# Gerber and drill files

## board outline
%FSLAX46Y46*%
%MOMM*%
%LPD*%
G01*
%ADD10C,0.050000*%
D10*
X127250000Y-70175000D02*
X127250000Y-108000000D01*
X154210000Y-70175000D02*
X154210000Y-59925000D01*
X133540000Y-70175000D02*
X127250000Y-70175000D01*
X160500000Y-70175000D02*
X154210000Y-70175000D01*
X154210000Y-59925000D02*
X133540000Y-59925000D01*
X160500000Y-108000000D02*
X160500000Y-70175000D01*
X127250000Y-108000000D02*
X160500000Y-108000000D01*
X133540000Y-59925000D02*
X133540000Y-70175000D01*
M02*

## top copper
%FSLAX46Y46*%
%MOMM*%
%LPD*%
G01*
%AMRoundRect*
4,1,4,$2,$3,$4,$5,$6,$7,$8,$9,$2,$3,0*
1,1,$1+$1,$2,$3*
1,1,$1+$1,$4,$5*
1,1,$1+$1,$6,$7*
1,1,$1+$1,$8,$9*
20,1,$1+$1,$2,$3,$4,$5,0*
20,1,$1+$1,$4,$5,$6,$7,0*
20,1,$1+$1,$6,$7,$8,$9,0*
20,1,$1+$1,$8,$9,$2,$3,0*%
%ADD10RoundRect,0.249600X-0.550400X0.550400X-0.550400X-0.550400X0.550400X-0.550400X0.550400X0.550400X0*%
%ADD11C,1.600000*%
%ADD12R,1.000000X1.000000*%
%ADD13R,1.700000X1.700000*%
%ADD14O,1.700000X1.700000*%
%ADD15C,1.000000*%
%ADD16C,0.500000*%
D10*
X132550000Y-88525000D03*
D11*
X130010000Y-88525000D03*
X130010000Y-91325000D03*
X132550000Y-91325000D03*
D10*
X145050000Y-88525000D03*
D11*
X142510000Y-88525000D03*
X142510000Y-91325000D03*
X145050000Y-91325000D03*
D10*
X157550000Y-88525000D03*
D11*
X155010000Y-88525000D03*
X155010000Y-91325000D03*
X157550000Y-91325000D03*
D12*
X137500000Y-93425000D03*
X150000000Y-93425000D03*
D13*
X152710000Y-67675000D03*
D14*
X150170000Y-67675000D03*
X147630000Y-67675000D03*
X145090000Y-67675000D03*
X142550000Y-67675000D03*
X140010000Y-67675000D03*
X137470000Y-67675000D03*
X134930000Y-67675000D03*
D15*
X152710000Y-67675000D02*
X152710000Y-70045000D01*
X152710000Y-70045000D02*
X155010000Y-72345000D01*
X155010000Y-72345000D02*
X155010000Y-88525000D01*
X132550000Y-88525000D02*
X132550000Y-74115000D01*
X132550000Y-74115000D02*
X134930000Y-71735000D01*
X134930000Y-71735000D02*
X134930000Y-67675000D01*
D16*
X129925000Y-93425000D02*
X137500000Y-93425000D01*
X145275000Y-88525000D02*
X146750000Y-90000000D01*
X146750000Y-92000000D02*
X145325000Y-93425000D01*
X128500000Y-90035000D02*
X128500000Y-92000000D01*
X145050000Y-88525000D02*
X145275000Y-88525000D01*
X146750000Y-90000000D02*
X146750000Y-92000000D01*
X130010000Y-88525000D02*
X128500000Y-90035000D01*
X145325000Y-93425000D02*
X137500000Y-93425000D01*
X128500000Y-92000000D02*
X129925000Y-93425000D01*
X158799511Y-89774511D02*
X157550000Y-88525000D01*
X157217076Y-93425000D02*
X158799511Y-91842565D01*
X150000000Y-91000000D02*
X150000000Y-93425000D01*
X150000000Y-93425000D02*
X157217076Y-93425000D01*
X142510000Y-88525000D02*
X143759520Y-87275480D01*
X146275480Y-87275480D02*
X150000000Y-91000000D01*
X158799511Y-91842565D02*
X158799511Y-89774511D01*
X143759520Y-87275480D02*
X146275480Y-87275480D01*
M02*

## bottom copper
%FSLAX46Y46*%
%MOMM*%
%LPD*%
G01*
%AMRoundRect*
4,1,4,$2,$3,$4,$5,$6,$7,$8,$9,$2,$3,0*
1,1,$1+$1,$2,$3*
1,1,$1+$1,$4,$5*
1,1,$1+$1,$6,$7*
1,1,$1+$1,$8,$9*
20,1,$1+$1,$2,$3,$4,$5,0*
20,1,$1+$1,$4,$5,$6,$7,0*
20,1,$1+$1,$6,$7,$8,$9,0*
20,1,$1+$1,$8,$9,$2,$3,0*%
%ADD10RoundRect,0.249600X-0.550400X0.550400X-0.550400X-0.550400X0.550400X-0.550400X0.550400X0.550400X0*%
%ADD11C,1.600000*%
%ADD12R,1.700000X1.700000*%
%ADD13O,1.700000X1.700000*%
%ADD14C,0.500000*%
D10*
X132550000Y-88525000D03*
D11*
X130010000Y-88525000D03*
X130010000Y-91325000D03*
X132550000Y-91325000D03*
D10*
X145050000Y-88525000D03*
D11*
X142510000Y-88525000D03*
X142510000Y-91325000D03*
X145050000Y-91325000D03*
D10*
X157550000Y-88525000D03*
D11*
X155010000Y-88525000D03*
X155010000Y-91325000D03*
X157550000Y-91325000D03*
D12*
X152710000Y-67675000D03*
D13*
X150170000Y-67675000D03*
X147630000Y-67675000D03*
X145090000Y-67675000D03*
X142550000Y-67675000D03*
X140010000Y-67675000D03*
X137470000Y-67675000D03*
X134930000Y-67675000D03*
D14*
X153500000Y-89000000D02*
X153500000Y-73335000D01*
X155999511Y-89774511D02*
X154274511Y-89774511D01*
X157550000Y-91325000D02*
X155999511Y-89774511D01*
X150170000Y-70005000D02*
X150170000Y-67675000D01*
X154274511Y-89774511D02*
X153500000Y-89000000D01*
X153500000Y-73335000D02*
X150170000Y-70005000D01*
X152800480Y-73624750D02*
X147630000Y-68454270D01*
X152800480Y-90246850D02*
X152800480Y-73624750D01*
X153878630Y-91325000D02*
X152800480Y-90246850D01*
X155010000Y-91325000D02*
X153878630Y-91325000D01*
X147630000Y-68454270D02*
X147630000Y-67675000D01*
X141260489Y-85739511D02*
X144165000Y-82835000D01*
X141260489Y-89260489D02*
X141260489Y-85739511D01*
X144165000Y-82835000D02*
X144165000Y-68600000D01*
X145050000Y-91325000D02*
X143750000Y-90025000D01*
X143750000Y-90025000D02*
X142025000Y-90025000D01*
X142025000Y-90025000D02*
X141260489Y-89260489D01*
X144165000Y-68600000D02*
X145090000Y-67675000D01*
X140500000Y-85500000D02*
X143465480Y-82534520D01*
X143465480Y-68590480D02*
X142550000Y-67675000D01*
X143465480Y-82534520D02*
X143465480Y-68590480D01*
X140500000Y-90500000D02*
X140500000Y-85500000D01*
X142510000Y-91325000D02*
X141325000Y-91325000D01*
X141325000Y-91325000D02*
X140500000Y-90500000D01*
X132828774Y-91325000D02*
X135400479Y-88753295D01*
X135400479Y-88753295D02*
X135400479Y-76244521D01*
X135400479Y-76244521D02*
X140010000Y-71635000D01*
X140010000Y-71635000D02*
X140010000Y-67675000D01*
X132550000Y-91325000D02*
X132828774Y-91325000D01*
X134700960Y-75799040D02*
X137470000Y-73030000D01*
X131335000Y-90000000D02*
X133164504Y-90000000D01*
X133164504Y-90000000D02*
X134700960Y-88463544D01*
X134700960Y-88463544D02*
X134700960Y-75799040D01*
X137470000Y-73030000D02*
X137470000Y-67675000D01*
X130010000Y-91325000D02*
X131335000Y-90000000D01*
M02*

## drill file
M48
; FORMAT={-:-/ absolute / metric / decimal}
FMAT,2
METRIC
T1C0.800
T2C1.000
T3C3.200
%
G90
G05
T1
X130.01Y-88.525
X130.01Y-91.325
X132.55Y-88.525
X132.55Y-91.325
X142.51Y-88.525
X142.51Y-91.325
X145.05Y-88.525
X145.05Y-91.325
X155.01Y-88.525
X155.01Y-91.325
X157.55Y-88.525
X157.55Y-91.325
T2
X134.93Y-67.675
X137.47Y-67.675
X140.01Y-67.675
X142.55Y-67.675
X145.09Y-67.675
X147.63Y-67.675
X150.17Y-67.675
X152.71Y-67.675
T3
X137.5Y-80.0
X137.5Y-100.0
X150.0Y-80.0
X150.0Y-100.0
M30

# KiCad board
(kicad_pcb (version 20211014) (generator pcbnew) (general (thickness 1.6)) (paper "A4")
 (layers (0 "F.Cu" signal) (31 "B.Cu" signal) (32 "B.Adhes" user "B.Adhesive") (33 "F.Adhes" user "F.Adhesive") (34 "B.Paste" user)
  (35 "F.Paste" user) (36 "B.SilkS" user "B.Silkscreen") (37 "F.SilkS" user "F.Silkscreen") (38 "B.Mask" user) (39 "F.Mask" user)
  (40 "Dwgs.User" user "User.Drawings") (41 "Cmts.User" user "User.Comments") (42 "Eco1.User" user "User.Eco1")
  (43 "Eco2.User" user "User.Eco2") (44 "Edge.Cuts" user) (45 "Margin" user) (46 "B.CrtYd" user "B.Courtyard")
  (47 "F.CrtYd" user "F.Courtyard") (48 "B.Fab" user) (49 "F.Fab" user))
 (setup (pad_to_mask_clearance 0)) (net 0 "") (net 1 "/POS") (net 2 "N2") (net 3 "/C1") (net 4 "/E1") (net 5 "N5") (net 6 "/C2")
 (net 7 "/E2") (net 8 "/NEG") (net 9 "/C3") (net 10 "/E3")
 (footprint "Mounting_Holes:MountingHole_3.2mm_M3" (layer "F.Cu") (at 137.5 100)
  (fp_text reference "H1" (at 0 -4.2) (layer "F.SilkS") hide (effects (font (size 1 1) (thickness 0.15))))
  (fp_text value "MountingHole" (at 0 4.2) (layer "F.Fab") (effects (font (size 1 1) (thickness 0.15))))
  (pad "" np_thru_hole circle locked (at 0 0) (size 3.2 3.2) (drill 3.2) (layers *.Cu *.Mask)))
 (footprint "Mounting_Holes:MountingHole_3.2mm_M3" (layer "F.Cu") (at 137.5 80)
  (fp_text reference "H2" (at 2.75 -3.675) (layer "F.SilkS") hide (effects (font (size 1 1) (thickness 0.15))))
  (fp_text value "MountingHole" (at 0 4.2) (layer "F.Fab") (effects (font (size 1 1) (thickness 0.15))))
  (pad "" np_thru_hole circle locked (at 0 0) (size 3.2 3.2) (drill 3.2) (layers *.Cu *.Mask)))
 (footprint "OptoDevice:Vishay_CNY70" (layer "F.Cu") (at 132.55 88.525 -90)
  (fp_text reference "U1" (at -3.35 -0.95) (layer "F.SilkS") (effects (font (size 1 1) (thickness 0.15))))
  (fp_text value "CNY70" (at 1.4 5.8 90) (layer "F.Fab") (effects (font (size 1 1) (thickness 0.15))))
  (pad "1" thru_hole roundrect (at 0 0 270) (size 1.6 1.6) (drill 0.8) (layers *.Cu *.Mask) (roundrect_rratio 0.156) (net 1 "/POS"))
  (pad "2" thru_hole circle (at 0 2.54 270) (size 1.6 1.6) (drill 0.8) (layers *.Cu *.Mask) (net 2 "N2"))
  (pad "3" thru_hole circle (at 2.8 2.54 270) (size 1.6 1.6) (drill 0.8) (layers *.Cu *.Mask) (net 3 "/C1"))
  (pad "4" thru_hole circle (at 2.8 0 270) (size 1.6 1.6) (drill 0.8) (layers *.Cu *.Mask) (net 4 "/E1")))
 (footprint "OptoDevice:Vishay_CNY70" (layer "F.Cu") (at 145.05 88.525 -90)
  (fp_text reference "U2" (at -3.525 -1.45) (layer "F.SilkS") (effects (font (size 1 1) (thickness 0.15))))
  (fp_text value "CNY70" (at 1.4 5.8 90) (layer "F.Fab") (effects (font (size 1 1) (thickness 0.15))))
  (pad "1" thru_hole roundrect (at 0 0 270) (size 1.6 1.6) (drill 0.8) (layers *.Cu *.Mask) (roundrect_rratio 0.156) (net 2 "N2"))
  (pad "2" thru_hole circle (at 0 2.54 270) (size 1.6 1.6) (drill 0.8) (layers *.Cu *.Mask) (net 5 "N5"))
  (pad "3" thru_hole circle (at 2.8 2.54 270) (size 1.6 1.6) (drill 0.8) (layers *.Cu *.Mask) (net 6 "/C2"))
  (pad "4" thru_hole circle (at 2.8 0 270) (size 1.6 1.6) (drill 0.8) (layers *.Cu *.Mask) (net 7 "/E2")))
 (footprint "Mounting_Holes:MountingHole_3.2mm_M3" (layer "F.Cu") (at 150 100)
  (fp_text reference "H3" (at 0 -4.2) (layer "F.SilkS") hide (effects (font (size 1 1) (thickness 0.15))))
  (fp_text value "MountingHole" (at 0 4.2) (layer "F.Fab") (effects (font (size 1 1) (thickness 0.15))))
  (pad "" np_thru_hole circle locked (at 0 0) (size 3.2 3.2) (drill 3.2) (layers *.Cu *.Mask)))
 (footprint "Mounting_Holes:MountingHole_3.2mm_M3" (layer "F.Cu") (at 150 80)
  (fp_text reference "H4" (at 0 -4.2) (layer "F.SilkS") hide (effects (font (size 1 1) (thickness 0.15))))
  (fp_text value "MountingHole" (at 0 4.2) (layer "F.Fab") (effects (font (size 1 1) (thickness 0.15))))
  (pad "" np_thru_hole circle locked (at 0 0) (size 3.2 3.2) (drill 3.2) (layers *.Cu *.Mask)))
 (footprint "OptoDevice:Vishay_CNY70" (layer "F.Cu") (at 157.55 88.525 -90)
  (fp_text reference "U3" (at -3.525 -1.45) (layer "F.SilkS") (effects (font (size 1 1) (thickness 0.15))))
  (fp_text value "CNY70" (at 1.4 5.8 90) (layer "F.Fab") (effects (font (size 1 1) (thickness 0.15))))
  (pad "1" thru_hole roundrect (at 0 0 270) (size 1.6 1.6) (drill 0.8) (layers *.Cu *.Mask) (roundrect_rratio 0.156) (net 5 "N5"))
  (pad "2" thru_hole circle (at 0 2.54 270) (size 1.6 1.6) (drill 0.8) (layers *.Cu *.Mask) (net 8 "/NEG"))
  (pad "3" thru_hole circle (at 2.8 2.54 270) (size 1.6 1.6) (drill 0.8) (layers *.Cu *.Mask) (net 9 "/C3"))
  (pad "4" thru_hole circle (at 2.8 0 270) (size 1.6 1.6) (drill 0.8) (layers *.Cu *.Mask) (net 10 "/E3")))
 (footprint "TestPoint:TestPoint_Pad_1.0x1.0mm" (layer "F.Cu") (at 137.5 93.425)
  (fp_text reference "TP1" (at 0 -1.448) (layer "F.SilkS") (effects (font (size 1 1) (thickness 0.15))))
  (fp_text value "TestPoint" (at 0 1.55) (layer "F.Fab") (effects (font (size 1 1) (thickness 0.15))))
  (pad "1" smd rect locked (at 0 0) (size 1 1) (layers "F.Cu" "F.Mask") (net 2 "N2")))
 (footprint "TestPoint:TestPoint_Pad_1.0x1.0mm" (layer "F.Cu") (at 150 93.425)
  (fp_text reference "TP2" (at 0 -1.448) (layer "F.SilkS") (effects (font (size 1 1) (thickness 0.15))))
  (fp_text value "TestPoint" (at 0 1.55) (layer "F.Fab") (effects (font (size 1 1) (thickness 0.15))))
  (pad "1" smd rect locked (at 0 0) (size 1 1) (layers "F.Cu" "F.Mask") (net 5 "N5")))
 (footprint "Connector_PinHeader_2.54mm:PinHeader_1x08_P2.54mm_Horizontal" (layer "B.Cu") (at 152.71 67.675 90)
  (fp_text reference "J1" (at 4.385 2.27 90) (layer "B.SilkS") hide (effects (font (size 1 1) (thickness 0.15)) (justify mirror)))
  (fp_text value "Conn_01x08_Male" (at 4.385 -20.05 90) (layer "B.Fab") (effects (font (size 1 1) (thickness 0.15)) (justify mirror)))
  (pad "1" thru_hole rect (at 0 0 90) (size 1.7 1.7) (drill 1) (layers *.Cu *.Mask) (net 8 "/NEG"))
  (pad "2" thru_hole oval (at 0 -2.54 90) (size 1.7 1.7) (drill 1) (layers *.Cu *.Mask) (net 10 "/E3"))
  (pad "3" thru_hole oval (at 0 -5.08 90) (size 1.7 1.7) (drill 1) (layers *.Cu *.Mask) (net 9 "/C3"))
  (pad "4" thru_hole oval (at 0 -7.62 90) (size 1.7 1.7) (drill 1) (layers *.Cu *.Mask) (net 7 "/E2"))
  (pad "5" thru_hole oval (at 0 -10.16 90) (size 1.7 1.7) (drill 1) (layers *.Cu *.Mask) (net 6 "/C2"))
  (pad "6" thru_hole oval (at 0 -12.7 90) (size 1.7 1.7) (drill 1) (layers *.Cu *.Mask) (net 4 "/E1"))
  (pad "7" thru_hole oval (at 0 -15.24 90) (size 1.7 1.7) (drill 1) (layers *.Cu *.Mask) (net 3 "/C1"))
  (pad "8" thru_hole oval (at 0 -17.78 90) (size 1.7 1.7) (drill 1) (layers *.Cu *.Mask) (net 1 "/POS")))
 (gr_line (start 127.25 70.175) (end 127.25 108) (layer "Edge.Cuts") (width 0.05))
 (gr_line (start 154.21 70.175) (end 154.21 59.925) (layer "Edge.Cuts") (width 0.05))
 (gr_line (start 133.54 70.175) (end 127.25 70.175) (layer "Edge.Cuts") (width 0.05))
 (gr_line (start 160.5 70.175) (end 154.21 70.175) (layer "Edge.Cuts") (width 0.05))
 (gr_line (start 154.21 59.925) (end 133.54 59.925) (layer "Edge.Cuts") (width 0.05))
 (gr_line (start 160.5 108) (end 160.5 70.175) (layer "Edge.Cuts") (width 0.05))
 (gr_line (start 127.25 108) (end 160.5 108) (layer "Edge.Cuts") (width 0.05))
 (gr_line (start 133.54 59.925) (end 133.54 70.175) (layer "Edge.Cuts") (width 0.05))
 (segment (start 152.71 67.675) (end 152.71 70.045) (width 1) (layer "F.Cu") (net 8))
 (segment (start 152.71 70.045) (end 155.01 72.345) (width 1) (layer "F.Cu") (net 8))
 (segment (start 155.01 72.345) (end 155.01 88.525) (width 1) (layer "F.Cu") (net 8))
 (segment (start 132.55 88.525) (end 132.55 74.115) (width 1) (layer "F.Cu") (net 1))
 (segment (start 132.55 74.115) (end 134.93 71.735) (width 1) (layer "F.Cu") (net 1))
 (segment (start 134.93 71.735) (end 134.93 67.675) (width 1) (layer "F.Cu") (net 1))
 (segment (start 153.5 89) (end 153.5 73.335) (width 0.5) (layer "B.Cu") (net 10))
 (segment (start 155.999511 89.774511) (end 154.274511 89.774511) (width 0.5) (layer "B.Cu") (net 10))
 (segment (start 157.55 91.325) (end 155.999511 89.774511) (width 0.5) (layer "B.Cu") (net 10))
 (segment (start 150.17 70.005) (end 150.17 67.675) (width 0.5) (layer "B.Cu") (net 10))
 (segment (start 154.274511 89.774511) (end 153.5 89) (width 0.5) (layer "B.Cu") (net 10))
 (segment (start 153.5 73.335) (end 150.17 70.005) (width 0.5) (layer "B.Cu") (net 10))
 (segment (start 152.80048 73.62475) (end 147.63 68.45427) (width 0.5) (layer "B.Cu") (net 9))
 (segment (start 152.80048 90.24685) (end 152.80048 73.62475) (width 0.5) (layer "B.Cu") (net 9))
 (segment (start 153.87863 91.325) (end 152.80048 90.24685) (width 0.5) (layer "B.Cu") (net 9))
 (segment (start 155.01 91.325) (end 153.87863 91.325) (width 0.5) (layer "B.Cu") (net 9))
 (segment (start 147.63 68.45427) (end 147.63 67.675) (width 0.5) (layer "B.Cu") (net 9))
 (segment (start 141.260489 85.739511) (end 144.165 82.835) (width 0.5) (layer "B.Cu") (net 7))
 (segment (start 141.260489 89.260489) (end 141.260489 85.739511) (width 0.5) (layer "B.Cu") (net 7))
 (segment (start 144.165 82.835) (end 144.165 68.6) (width 0.5) (layer "B.Cu") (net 7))
 (segment (start 145.05 91.325) (end 143.75 90.025) (width 0.5) (layer "B.Cu") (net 7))
 (segment (start 143.75 90.025) (end 142.025 90.025) (width 0.5) (layer "B.Cu") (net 7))
 (segment (start 142.025 90.025) (end 141.260489 89.260489) (width 0.5) (layer "B.Cu") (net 7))
 (segment (start 144.165 68.6) (end 145.09 67.675) (width 0.5) (layer "B.Cu") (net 7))
 (segment (start 140.5 85.5) (end 143.46548 82.53452) (width 0.5) (layer "B.Cu") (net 6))
 (segment (start 143.46548 68.59048) (end 142.55 67.675) (width 0.5) (layer "B.Cu") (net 6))
 (segment (start 143.46548 82.53452) (end 143.46548 68.59048) (width 0.5) (layer "B.Cu") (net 6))
 (segment (start 140.5 90.5) (end 140.5 85.5) (width 0.5) (layer "B.Cu") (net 6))
 (segment (start 142.51 91.325) (end 141.325 91.325) (width 0.5) (layer "B.Cu") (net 6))
 (segment (start 141.325 91.325) (end 140.5 90.5) (width 0.5) (layer "B.Cu") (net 6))
 (segment (start 132.828774 91.325) (end 135.400479 88.753295) (width 0.5) (layer "B.Cu") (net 4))
 (segment (start 135.400479 88.753295) (end 135.400479 76.244521) (width 0.5) (layer "B.Cu") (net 4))
 (segment (start 135.400479 76.244521) (end 140.01 71.635) (width 0.5) (layer "B.Cu") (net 4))
 (segment (start 140.01 71.635) (end 140.01 67.675) (width 0.5) (layer "B.Cu") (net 4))
 (segment (start 132.55 91.325) (end 132.828774 91.325) (width 0.5) (layer "B.Cu") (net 4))
 (segment (start 134.70096 75.79904) (end 137.47 73.03) (width 0.5) (layer "B.Cu") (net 3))
 (segment (start 131.335 90) (end 133.164504 90) (width 0.5) (layer "B.Cu") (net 3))
 (segment (start 133.164504 90) (end 134.70096 88.463544) (width 0.5) (layer "B.Cu") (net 3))
 (segment (start 134.70096 88.463544) (end 134.70096 75.79904) (width 0.5) (layer "B.Cu") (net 3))
 (segment (start 137.47 73.03) (end 137.47 67.675) (width 0.5) (layer "B.Cu") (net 3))
 (segment (start 130.01 91.325) (end 131.335 90) (width 0.5) (layer "B.Cu") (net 3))
 (segment (start 129.925 93.425) (end 137.5 93.425) (width 0.5) (layer "F.Cu") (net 2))
 (segment (start 145.275 88.525) (end 146.75 90) (width 0.5) (layer "F.Cu") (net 2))
 (segment (start 146.75 92) (end 145.325 93.425) (width 0.5) (layer "F.Cu") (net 2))
 (segment (start 128.5 90.035) (end 128.5 92) (width 0.5) (layer "F.Cu") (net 2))
 (segment (start 145.05 88.525) (end 145.275 88.525) (width 0.5) (layer "F.Cu") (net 2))
 (segment (start 146.75 90) (end 146.75 92) (width 0.5) (layer "F.Cu") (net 2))
 (segment (start 130.01 88.525) (end 128.5 90.035) (width 0.5) (layer "F.Cu") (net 2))
 (segment (start 145.325 93.425) (end 137.5 93.425) (width 0.5) (layer "F.Cu") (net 2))
 (segment (start 128.5 92) (end 129.925 93.425) (width 0.5) (layer "F.Cu") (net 2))
 (segment (start 158.799511 89.774511) (end 157.55 88.525) (width 0.5) (layer "F.Cu") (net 5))
 (segment (start 157.217076 93.425) (end 158.799511 91.842565) (width 0.5) (layer "F.Cu") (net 5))
 (segment (start 150 91) (end 150 93.425) (width 0.5) (layer "F.Cu") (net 5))
 (segment (start 150 93.425) (end 157.217076 93.425) (width 0.5) (layer "F.Cu") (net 5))
 (segment (start 142.51 88.525) (end 143.75952 87.27548) (width 0.5) (layer "F.Cu") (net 5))
 (segment (start 146.27548 87.27548) (end 150 91) (width 0.5) (layer "F.Cu") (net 5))
 (segment (start 158.799511 91.842565) (end 158.799511 89.774511) (width 0.5) (layer "F.Cu") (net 5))
 (segment (start 143.75952 87.27548) (end 146.27548 87.27548) (width 0.5) (layer "F.Cu") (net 5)))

